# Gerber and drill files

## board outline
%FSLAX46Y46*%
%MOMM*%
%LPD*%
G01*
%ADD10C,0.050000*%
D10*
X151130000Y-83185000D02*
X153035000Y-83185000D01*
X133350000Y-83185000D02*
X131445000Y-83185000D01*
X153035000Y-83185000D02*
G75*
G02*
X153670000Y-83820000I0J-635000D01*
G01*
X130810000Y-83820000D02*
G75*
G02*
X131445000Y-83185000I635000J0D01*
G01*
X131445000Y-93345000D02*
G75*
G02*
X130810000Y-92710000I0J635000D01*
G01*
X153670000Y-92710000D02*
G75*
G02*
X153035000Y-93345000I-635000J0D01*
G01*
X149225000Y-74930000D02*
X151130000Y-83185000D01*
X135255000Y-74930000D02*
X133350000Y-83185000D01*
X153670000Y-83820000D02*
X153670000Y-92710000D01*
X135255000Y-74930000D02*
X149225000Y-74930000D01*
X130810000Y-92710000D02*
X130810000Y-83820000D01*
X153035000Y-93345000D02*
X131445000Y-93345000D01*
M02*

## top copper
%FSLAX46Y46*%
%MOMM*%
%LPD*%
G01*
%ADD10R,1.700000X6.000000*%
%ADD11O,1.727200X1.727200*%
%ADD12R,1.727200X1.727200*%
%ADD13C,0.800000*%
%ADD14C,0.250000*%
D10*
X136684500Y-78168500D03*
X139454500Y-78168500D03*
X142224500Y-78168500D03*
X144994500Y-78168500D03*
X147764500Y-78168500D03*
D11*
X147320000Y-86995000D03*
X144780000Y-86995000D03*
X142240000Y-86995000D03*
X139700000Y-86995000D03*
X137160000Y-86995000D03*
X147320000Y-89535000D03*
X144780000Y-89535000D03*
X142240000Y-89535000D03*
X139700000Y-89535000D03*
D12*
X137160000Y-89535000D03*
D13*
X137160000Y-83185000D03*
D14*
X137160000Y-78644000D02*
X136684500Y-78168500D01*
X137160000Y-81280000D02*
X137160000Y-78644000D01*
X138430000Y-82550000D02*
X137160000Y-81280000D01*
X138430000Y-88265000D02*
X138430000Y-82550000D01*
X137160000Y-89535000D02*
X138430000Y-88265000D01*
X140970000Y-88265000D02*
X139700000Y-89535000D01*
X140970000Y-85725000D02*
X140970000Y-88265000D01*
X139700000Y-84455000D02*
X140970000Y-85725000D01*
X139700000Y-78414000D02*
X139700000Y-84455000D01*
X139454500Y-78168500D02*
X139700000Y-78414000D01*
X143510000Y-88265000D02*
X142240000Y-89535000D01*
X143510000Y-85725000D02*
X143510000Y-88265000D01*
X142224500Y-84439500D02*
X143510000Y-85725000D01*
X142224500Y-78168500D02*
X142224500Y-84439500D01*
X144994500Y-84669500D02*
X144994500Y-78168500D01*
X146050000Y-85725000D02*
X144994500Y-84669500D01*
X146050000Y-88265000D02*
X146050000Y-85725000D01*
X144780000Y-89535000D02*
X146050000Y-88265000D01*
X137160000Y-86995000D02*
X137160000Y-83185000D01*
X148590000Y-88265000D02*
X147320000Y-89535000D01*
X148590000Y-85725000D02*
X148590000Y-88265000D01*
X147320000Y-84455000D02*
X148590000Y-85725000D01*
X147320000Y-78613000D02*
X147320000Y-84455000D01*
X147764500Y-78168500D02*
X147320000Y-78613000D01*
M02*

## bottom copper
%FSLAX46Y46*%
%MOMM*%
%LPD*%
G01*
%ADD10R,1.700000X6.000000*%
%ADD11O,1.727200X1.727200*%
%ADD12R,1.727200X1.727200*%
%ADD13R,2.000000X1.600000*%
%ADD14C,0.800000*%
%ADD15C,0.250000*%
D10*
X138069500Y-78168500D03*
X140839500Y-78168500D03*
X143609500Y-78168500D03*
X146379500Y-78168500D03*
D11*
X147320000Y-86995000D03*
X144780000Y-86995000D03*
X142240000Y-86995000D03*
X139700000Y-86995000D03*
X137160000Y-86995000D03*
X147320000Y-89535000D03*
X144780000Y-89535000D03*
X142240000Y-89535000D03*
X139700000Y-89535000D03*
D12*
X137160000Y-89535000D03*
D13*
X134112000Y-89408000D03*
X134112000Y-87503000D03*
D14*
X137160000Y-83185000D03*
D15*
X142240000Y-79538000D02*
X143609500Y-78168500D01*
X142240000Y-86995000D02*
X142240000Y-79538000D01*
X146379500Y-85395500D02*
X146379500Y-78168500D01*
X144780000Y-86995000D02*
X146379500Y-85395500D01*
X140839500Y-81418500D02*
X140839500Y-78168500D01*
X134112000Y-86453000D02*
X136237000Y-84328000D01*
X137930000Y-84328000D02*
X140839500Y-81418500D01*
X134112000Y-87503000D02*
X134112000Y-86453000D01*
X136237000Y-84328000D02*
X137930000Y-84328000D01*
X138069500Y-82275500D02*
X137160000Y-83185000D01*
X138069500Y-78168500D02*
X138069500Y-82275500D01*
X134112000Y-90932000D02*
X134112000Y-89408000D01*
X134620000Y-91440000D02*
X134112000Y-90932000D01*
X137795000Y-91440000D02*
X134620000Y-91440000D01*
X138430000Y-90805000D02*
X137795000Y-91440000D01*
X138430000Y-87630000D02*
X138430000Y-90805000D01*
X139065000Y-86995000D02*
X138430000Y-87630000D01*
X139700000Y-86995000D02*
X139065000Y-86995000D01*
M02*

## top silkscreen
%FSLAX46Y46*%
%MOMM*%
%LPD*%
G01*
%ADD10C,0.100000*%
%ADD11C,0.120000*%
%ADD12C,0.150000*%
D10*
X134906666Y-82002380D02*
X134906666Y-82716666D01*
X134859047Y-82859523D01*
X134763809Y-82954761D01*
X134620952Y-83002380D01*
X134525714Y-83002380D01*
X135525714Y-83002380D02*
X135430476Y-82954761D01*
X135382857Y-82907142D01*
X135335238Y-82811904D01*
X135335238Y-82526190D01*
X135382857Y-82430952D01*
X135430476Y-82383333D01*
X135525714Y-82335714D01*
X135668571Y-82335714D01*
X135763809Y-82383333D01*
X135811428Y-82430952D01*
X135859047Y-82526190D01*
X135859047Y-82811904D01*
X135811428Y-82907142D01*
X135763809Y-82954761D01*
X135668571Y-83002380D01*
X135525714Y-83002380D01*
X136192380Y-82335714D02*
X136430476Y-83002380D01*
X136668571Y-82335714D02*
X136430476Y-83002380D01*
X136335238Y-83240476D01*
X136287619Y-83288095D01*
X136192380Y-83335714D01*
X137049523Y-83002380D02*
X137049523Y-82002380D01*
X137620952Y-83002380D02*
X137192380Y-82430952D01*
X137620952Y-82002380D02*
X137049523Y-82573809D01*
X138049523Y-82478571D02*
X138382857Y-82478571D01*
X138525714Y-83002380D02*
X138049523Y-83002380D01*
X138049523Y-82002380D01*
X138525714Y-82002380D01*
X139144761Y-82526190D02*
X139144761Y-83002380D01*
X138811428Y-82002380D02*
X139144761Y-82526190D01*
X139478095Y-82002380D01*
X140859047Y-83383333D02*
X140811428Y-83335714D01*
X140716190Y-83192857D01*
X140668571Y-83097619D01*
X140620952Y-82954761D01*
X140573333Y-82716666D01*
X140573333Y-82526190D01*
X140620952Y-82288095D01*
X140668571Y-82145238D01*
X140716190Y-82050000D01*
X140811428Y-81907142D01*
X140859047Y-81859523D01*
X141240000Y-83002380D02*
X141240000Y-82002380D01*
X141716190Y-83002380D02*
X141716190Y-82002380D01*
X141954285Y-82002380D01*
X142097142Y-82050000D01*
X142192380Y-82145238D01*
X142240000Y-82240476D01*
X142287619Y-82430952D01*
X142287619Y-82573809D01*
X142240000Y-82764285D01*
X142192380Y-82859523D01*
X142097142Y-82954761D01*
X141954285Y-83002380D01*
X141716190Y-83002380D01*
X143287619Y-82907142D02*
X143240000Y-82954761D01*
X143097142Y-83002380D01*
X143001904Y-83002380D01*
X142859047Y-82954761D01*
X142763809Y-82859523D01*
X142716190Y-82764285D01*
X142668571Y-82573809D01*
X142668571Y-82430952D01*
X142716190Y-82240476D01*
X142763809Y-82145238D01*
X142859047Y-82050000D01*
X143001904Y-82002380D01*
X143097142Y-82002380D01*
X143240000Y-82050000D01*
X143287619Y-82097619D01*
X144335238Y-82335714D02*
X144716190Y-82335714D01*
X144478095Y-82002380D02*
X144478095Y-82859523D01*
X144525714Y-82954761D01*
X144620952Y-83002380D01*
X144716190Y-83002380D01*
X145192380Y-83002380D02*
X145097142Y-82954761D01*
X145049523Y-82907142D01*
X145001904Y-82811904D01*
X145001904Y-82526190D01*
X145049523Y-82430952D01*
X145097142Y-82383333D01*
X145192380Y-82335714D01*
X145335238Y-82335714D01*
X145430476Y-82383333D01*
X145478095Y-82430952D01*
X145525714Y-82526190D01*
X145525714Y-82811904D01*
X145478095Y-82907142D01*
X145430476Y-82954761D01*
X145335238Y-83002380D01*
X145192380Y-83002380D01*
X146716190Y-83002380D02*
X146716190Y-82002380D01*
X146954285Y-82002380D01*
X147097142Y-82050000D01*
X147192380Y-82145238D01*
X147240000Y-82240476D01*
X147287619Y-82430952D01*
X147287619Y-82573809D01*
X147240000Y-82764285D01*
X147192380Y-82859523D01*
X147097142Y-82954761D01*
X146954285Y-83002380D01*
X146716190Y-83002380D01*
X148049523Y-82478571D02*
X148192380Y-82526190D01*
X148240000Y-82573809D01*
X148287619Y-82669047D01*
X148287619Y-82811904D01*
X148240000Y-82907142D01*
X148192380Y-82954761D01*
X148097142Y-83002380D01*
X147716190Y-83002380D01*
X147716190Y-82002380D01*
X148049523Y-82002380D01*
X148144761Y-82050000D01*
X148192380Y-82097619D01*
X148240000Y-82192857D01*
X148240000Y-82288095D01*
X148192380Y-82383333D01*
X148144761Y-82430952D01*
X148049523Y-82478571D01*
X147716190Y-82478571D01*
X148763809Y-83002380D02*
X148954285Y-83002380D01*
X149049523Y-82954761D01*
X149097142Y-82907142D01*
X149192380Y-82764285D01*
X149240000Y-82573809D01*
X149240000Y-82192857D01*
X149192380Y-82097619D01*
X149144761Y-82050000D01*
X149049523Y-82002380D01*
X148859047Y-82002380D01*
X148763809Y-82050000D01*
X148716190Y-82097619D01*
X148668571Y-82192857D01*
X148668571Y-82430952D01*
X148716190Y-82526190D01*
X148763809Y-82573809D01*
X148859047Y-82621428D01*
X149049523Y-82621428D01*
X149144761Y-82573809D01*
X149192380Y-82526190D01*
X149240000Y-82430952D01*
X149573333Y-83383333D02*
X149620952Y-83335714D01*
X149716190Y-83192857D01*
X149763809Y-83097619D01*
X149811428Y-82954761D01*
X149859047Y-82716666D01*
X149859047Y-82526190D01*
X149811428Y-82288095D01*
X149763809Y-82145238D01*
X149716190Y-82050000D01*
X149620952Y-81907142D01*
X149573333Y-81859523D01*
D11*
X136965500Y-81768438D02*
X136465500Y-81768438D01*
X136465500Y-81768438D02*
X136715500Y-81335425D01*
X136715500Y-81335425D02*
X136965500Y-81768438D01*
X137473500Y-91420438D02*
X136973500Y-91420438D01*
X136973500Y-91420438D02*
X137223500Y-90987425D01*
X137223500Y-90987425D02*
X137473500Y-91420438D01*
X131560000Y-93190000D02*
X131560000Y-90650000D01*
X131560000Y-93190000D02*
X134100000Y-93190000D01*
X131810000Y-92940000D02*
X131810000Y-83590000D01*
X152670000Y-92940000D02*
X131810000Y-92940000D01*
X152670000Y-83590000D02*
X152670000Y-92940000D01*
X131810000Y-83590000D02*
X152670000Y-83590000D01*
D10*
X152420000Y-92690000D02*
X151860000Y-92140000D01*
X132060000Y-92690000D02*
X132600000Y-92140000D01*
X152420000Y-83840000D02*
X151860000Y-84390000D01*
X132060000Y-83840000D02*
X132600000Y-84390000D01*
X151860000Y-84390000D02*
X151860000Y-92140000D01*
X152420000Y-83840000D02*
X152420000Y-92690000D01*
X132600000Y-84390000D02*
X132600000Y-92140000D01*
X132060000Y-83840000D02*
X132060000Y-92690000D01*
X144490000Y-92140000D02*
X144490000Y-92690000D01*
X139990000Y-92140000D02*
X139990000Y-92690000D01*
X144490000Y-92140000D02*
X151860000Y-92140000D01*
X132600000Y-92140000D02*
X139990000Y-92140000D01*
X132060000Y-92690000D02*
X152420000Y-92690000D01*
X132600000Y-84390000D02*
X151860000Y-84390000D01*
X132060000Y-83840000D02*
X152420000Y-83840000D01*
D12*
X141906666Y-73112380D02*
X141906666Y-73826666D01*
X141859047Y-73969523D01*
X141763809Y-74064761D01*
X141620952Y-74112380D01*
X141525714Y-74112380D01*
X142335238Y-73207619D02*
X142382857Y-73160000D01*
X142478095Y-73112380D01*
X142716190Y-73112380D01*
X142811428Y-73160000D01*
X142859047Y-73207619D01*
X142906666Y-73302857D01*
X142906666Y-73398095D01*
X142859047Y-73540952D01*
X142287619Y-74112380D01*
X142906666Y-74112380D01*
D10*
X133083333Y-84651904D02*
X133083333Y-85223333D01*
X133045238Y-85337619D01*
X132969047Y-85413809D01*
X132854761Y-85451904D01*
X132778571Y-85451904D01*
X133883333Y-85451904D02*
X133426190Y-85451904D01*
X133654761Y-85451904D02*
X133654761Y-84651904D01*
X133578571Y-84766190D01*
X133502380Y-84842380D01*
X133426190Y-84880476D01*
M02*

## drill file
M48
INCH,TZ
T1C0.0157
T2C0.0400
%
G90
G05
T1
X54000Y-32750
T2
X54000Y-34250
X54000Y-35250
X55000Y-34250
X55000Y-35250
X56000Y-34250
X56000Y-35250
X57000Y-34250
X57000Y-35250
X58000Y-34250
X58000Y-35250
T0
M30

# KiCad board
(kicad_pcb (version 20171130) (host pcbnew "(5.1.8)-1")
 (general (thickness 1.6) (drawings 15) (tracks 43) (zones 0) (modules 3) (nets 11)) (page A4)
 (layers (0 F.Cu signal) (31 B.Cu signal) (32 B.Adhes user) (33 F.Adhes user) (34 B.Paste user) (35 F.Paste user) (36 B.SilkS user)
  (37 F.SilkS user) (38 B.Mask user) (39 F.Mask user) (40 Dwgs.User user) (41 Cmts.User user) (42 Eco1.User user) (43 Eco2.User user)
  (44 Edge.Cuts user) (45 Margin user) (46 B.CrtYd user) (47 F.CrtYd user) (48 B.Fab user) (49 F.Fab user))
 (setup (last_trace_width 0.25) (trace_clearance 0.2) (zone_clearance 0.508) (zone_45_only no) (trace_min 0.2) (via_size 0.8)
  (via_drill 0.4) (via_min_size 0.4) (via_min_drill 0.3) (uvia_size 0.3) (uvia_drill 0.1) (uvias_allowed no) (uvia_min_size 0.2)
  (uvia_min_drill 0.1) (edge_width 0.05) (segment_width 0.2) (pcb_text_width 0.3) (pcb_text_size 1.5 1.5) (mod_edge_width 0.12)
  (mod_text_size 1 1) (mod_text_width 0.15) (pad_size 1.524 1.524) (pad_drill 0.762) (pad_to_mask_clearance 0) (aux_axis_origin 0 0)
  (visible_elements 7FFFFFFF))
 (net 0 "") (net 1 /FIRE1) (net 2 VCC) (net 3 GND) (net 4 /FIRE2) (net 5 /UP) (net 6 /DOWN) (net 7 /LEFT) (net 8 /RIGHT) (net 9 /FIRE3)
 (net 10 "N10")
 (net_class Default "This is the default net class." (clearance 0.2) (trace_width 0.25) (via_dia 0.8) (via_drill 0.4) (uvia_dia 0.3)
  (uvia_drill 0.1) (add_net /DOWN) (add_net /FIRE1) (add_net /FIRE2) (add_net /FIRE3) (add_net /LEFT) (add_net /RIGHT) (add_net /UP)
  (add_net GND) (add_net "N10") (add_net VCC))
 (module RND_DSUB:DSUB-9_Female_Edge (layer F.Cu) (at 142.24 78.105)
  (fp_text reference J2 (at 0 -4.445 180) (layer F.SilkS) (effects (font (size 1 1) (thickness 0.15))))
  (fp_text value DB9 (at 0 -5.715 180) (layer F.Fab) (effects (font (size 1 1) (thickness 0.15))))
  (fp_line (start -5.2745 3.663438) (end -5.7745 3.663438) (layer F.SilkS) (width 0.12))
  (fp_line (start -5.7745 3.663438) (end -5.5245 3.230425) (layer F.SilkS) (width 0.12))
  (fp_line (start -5.5245 3.230425) (end -5.2745 3.663438) (layer F.SilkS) (width 0.12))
  (pad 6 smd rect (at -4.1705 0.0635 180) (size 1.7 6) (layers B.Cu B.Paste B.Mask) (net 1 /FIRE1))
  (pad 7 smd rect (at -1.4005 0.0635 180) (size 1.7 6) (layers B.Cu B.Paste B.Mask) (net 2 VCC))
  (pad 8 smd rect (at 1.3695 0.0635 180) (size 1.7 6) (layers B.Cu B.Paste B.Mask) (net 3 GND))
  (pad 9 smd rect (at 4.1395 0.0635 180) (size 1.7 6) (layers B.Cu B.Paste B.Mask) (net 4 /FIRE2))
  (pad 1 smd rect (at -5.5555 0.0635 180) (size 1.7 6) (layers F.Cu F.Paste F.Mask) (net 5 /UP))
  (pad 2 smd rect (at -2.7855 0.0635 180) (size 1.7 6) (layers F.Cu F.Paste F.Mask) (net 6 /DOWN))
  (pad 3 smd rect (at -0.0155 0.0635 180) (size 1.7 6) (layers F.Cu F.Paste F.Mask) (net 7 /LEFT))
  (pad 4 smd rect (at 2.7545 0.0635 180) (size 1.7 6) (layers F.Cu F.Paste F.Mask) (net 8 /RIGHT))
  (pad 5 smd rect (at 5.5245 0.0635 180) (size 1.7 6) (layers F.Cu F.Paste F.Mask) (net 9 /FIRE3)))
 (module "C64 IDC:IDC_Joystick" (layer F.Cu) (at 137.16 89.535 90)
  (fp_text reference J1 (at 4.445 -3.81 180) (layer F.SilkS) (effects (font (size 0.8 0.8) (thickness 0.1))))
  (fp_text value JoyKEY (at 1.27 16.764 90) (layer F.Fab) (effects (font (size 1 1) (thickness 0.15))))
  (fp_line (start -1.885438 0.3135) (end -1.885438 -0.1865) (layer F.SilkS) (width 0.12))
  (fp_line (start -1.885438 -0.1865) (end -1.452425 0.0635) (layer F.SilkS) (width 0.12))
  (fp_line (start -1.452425 0.0635) (end -1.885438 0.3135) (layer F.SilkS) (width 0.12))
  (fp_line (start -3.655 -5.6) (end -1.115 -5.6) (layer F.SilkS) (width 0.12))
  (fp_line (start -3.655 -5.6) (end -3.655 -3.06) (layer F.SilkS) (width 0.12))
  (fp_line (start -3.405 -5.35) (end 5.945 -5.35) (layer F.SilkS) (width 0.12))
  (fp_line (start -3.405 15.51) (end -3.405 -5.35) (layer F.SilkS) (width 0.12))
  (fp_line (start 5.945 15.51) (end -3.405 15.51) (layer F.SilkS) (width 0.12))
  (fp_line (start 5.945 -5.35) (end 5.945 15.51) (layer F.SilkS) (width 0.12))
  (fp_line (start -3.155 15.26) (end -2.605 14.7) (layer F.SilkS) (width 0.1))
  (fp_line (start -3.155 -5.1) (end -2.605 -4.56) (layer F.SilkS) (width 0.1))
  (fp_line (start 5.695 15.26) (end 5.145 14.7) (layer F.SilkS) (width 0.1))
  (fp_line (start 5.695 -5.1) (end 5.145 -4.56) (layer F.SilkS) (width 0.1))
  (fp_line (start 5.145 14.7) (end -2.605 14.7) (layer F.SilkS) (width 0.1))
  (fp_line (start 5.695 15.26) (end -3.155 15.26) (layer F.SilkS) (width 0.1))
  (fp_line (start 5.145 -4.56) (end -2.605 -4.56) (layer F.SilkS) (width 0.1))
  (fp_line (start 5.695 -5.1) (end -3.155 -5.1) (layer F.SilkS) (width 0.1))
  (fp_line (start -2.605 7.33) (end -3.155 7.33) (layer F.SilkS) (width 0.1))
  (fp_line (start -2.605 2.83) (end -3.155 2.83) (layer F.SilkS) (width 0.1))
  (fp_line (start -2.605 7.33) (end -2.605 14.7) (layer F.SilkS) (width 0.1))
  (fp_line (start -2.605 -4.56) (end -2.605 2.83) (layer F.SilkS) (width 0.1))
  (fp_line (start -3.155 -5.1) (end -3.155 15.26) (layer F.SilkS) (width 0.1))
  (fp_line (start 5.145 -4.56) (end 5.145 14.7) (layer F.SilkS) (width 0.1))
  (fp_line (start 5.695 -5.1) (end 5.695 15.26) (layer F.SilkS) (width 0.1))
  (pad 10 thru_hole oval (at 2.54 10.16 90) (size 1.7272 1.7272) (drill 1.016) (layers *.Cu *.Mask))
  (pad 9 thru_hole oval (at 2.54 7.62 90) (size 1.7272 1.7272) (drill 1.016) (layers *.Cu *.Mask) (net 4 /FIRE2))
  (pad 8 thru_hole oval (at 2.54 5.08 90) (size 1.7272 1.7272) (drill 1.016) (layers *.Cu *.Mask) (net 3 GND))
  (pad 7 thru_hole oval (at 2.54 2.54 90) (size 1.7272 1.7272) (drill 1.016) (layers *.Cu *.Mask) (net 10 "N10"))
  (pad 6 thru_hole oval (at 2.54 0 90) (size 1.7272 1.7272) (drill 1.016) (layers *.Cu *.Mask) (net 1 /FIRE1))
  (pad 5 thru_hole oval (at 0 10.16 90) (size 1.7272 1.7272) (drill 1.016) (layers *.Cu *.Mask) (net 9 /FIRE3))
  (pad 4 thru_hole oval (at 0 7.62 90) (size 1.7272 1.7272) (drill 1.016) (layers *.Cu *.Mask) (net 8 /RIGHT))
  (pad 3 thru_hole oval (at 0 5.08 90) (size 1.7272 1.7272) (drill 1.016) (layers *.Cu *.Mask) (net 7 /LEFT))
  (pad 2 thru_hole oval (at 0 2.54 90) (size 1.7272 1.7272) (drill 1.016) (layers *.Cu *.Mask) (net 6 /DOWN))
  (pad 1 thru_hole rect (at 0 0 90) (size 1.7272 1.7272) (drill 1.016) (layers *.Cu *.Mask) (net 5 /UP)))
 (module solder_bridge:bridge (layer B.Cu) (at 134.112 89.408)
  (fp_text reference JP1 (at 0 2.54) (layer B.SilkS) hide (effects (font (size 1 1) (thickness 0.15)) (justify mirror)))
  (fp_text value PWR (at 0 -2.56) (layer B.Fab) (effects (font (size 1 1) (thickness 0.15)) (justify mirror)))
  (pad 1 smd rect (at 0 0) (size 2 1.6) (layers B.Cu B.Paste B.Mask) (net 10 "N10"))
  (pad 2 smd rect (at 0 -1.905) (size 2 1.6) (layers B.Cu B.Paste B.Mask) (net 2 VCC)))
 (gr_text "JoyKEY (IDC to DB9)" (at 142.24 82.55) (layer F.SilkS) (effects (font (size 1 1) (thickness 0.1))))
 (gr_line (start 151.13 83.185) (end 153.035 83.185) (layer Edge.Cuts) (width 0.05))
 (gr_line (start 133.35 83.185) (end 131.445 83.185) (layer Edge.Cuts) (width 0.05))
 (gr_arc (start 153.035 83.82) (end 153.67 83.82) (angle -90) (layer Edge.Cuts) (width 0.05))
 (gr_arc (start 131.445 83.82) (end 131.445 83.185) (angle -90) (layer Edge.Cuts) (width 0.05))
 (gr_arc (start 131.445 92.71) (end 130.81 92.71) (angle -90) (layer Edge.Cuts) (width 0.05))
 (gr_arc (start 153.035 92.71) (end 153.035 93.345) (angle -90) (layer Edge.Cuts) (width 0.05))
 (gr_line (start 149.225 74.93) (end 151.13 83.185) (layer Edge.Cuts) (width 0.05))
 (gr_line (start 135.255 74.93) (end 133.35 83.185) (layer Edge.Cuts) (width 0.05))
 (gr_line (start 153.67 83.82) (end 153.67 92.71) (layer Edge.Cuts) (width 0.05))
 (gr_line (start 135.255 74.93) (end 149.225 74.93) (layer Edge.Cuts) (width 0.05))
 (gr_line (start 130.81 92.71) (end 130.81 83.82) (layer Edge.Cuts) (width 0.05))
 (gr_line (start 153.035 93.345) (end 131.445 93.345) (layer Edge.Cuts) (width 0.05))
 (segment (start 142.24 79.538) (end 143.6095 78.1685) (width 0.25) (layer B.Cu) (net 3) (status 20))
 (segment (start 142.24 86.995) (end 142.24 79.538) (width 0.25) (layer B.Cu) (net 3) (status 10))
 (segment (start 137.16 78.644) (end 136.6845 78.1685) (width 0.25) (layer F.Cu) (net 5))
 (segment (start 137.16 81.28) (end 137.16 78.644) (width 0.25) (layer F.Cu) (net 5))
 (segment (start 138.43 82.55) (end 137.16 81.28) (width 0.25) (layer F.Cu) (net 5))
 (segment (start 138.43 88.265) (end 138.43 82.55) (width 0.25) (layer F.Cu) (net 5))
 (segment (start 137.16 89.535) (end 138.43 88.265) (width 0.25) (layer F.Cu) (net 5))
 (segment (start 140.97 88.265) (end 139.7 89.535) (width 0.25) (layer F.Cu) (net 6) (status 20))
 (segment (start 140.97 85.725) (end 140.97 88.265) (width 0.25) (layer F.Cu) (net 6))
 (segment (start 139.7 84.455) (end 140.97 85.725) (width 0.25) (layer F.Cu) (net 6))
 (segment (start 139.7 78.414) (end 139.7 84.455) (width 0.25) (layer F.Cu) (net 6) (status 10))
 (segment (start 139.4545 78.1685) (end 139.7 78.414) (width 0.25) (layer F.Cu) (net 6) (status 30))
 (segment (start 143.51 88.265) (end 142.24 89.535) (width 0.25) (layer F.Cu) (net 7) (status 20))
 (segment (start 143.51 85.725) (end 143.51 88.265) (width 0.25) (layer F.Cu) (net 7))
 (segment (start 142.2245 84.4395) (end 143.51 85.725) (width 0.25) (layer F.Cu) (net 7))
 (segment (start 142.2245 78.1685) (end 142.2245 84.4395) (width 0.25) (layer F.Cu) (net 7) (status 10))
 (segment (start 144.9945 84.6695) (end 144.9945 78.1685) (width 0.25) (layer F.Cu) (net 8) (status 20))
 (segment (start 146.05 85.725) (end 144.9945 84.6695) (width 0.25) (layer F.Cu) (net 8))
 (segment (start 146.05 88.265) (end 146.05 85.725) (width 0.25) (layer F.Cu) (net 8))
 (segment (start 144.78 89.535) (end 146.05 88.265) (width 0.25) (layer F.Cu) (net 8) (status 10))
 (segment (start 146.3795 85.3955) (end 146.3795 78.1685) (width 0.25) (layer B.Cu) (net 4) (status 20))
 (segment (start 144.78 86.995) (end 146.3795 85.3955) (width 0.25) (layer B.Cu) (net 4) (status 10))
 (segment (start 140.8395 81.4185) (end 140.8395 78.1685) (width 0.25) (layer B.Cu) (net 2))
 (segment (start 134.112 86.453) (end 136.237 84.328) (width 0.25) (layer B.Cu) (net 2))
 (segment (start 137.93 84.328) (end 140.8395 81.4185) (width 0.25) (layer B.Cu) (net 2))
 (segment (start 134.112 87.503) (end 134.112 86.453) (width 0.25) (layer B.Cu) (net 2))
 (segment (start 136.237 84.328) (end 137.93 84.328) (width 0.25) (layer B.Cu) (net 2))
 (segment (start 138.0695 82.2755) (end 137.16 83.185) (width 0.25) (layer B.Cu) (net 1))
 (segment (start 138.0695 78.1685) (end 138.0695 82.2755) (width 0.25) (layer B.Cu) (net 1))
 (segment (start 137.16 86.995) (end 137.16 83.185) (width 0.25) (layer F.Cu) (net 1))
 (via (at 137.16 83.185) (size 0.8) (drill 0.4) (layers F.Cu B.Cu) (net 1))
 (segment (start 148.59 88.265) (end 147.32 89.535) (width 0.25) (layer F.Cu) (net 9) (status 20))
 (segment (start 148.59 85.725) (end 148.59 88.265) (width 0.25) (layer F.Cu) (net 9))
 (segment (start 147.32 84.455) (end 148.59 85.725) (width 0.25) (layer F.Cu) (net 9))
 (segment (start 147.32 78.613) (end 147.32 84.455) (width 0.25) (layer F.Cu) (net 9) (status 10))
 (segment (start 147.7645 78.1685) (end 147.32 78.613) (width 0.25) (layer F.Cu) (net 9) (status 30))
 (segment (start 134.112 90.932) (end 134.112 89.408) (width 0.25) (layer B.Cu) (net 10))
 (segment (start 134.62 91.44) (end 134.112 90.932) (width 0.25) (layer B.Cu) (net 10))
 (segment (start 137.795 91.44) (end 134.62 91.44) (width 0.25) (layer B.Cu) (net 10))
 (segment (start 138.43 90.805) (end 137.795 91.44) (width 0.25) (layer B.Cu) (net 10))
 (segment (start 138.43 87.63) (end 138.43 90.805) (width 0.25) (layer B.Cu) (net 10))
 (segment (start 139.065 86.995) (end 138.43 87.63) (width 0.25) (layer B.Cu) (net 10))
 (segment (start 139.7 86.995) (end 139.065 86.995) (width 0.25) (layer B.Cu) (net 10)))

